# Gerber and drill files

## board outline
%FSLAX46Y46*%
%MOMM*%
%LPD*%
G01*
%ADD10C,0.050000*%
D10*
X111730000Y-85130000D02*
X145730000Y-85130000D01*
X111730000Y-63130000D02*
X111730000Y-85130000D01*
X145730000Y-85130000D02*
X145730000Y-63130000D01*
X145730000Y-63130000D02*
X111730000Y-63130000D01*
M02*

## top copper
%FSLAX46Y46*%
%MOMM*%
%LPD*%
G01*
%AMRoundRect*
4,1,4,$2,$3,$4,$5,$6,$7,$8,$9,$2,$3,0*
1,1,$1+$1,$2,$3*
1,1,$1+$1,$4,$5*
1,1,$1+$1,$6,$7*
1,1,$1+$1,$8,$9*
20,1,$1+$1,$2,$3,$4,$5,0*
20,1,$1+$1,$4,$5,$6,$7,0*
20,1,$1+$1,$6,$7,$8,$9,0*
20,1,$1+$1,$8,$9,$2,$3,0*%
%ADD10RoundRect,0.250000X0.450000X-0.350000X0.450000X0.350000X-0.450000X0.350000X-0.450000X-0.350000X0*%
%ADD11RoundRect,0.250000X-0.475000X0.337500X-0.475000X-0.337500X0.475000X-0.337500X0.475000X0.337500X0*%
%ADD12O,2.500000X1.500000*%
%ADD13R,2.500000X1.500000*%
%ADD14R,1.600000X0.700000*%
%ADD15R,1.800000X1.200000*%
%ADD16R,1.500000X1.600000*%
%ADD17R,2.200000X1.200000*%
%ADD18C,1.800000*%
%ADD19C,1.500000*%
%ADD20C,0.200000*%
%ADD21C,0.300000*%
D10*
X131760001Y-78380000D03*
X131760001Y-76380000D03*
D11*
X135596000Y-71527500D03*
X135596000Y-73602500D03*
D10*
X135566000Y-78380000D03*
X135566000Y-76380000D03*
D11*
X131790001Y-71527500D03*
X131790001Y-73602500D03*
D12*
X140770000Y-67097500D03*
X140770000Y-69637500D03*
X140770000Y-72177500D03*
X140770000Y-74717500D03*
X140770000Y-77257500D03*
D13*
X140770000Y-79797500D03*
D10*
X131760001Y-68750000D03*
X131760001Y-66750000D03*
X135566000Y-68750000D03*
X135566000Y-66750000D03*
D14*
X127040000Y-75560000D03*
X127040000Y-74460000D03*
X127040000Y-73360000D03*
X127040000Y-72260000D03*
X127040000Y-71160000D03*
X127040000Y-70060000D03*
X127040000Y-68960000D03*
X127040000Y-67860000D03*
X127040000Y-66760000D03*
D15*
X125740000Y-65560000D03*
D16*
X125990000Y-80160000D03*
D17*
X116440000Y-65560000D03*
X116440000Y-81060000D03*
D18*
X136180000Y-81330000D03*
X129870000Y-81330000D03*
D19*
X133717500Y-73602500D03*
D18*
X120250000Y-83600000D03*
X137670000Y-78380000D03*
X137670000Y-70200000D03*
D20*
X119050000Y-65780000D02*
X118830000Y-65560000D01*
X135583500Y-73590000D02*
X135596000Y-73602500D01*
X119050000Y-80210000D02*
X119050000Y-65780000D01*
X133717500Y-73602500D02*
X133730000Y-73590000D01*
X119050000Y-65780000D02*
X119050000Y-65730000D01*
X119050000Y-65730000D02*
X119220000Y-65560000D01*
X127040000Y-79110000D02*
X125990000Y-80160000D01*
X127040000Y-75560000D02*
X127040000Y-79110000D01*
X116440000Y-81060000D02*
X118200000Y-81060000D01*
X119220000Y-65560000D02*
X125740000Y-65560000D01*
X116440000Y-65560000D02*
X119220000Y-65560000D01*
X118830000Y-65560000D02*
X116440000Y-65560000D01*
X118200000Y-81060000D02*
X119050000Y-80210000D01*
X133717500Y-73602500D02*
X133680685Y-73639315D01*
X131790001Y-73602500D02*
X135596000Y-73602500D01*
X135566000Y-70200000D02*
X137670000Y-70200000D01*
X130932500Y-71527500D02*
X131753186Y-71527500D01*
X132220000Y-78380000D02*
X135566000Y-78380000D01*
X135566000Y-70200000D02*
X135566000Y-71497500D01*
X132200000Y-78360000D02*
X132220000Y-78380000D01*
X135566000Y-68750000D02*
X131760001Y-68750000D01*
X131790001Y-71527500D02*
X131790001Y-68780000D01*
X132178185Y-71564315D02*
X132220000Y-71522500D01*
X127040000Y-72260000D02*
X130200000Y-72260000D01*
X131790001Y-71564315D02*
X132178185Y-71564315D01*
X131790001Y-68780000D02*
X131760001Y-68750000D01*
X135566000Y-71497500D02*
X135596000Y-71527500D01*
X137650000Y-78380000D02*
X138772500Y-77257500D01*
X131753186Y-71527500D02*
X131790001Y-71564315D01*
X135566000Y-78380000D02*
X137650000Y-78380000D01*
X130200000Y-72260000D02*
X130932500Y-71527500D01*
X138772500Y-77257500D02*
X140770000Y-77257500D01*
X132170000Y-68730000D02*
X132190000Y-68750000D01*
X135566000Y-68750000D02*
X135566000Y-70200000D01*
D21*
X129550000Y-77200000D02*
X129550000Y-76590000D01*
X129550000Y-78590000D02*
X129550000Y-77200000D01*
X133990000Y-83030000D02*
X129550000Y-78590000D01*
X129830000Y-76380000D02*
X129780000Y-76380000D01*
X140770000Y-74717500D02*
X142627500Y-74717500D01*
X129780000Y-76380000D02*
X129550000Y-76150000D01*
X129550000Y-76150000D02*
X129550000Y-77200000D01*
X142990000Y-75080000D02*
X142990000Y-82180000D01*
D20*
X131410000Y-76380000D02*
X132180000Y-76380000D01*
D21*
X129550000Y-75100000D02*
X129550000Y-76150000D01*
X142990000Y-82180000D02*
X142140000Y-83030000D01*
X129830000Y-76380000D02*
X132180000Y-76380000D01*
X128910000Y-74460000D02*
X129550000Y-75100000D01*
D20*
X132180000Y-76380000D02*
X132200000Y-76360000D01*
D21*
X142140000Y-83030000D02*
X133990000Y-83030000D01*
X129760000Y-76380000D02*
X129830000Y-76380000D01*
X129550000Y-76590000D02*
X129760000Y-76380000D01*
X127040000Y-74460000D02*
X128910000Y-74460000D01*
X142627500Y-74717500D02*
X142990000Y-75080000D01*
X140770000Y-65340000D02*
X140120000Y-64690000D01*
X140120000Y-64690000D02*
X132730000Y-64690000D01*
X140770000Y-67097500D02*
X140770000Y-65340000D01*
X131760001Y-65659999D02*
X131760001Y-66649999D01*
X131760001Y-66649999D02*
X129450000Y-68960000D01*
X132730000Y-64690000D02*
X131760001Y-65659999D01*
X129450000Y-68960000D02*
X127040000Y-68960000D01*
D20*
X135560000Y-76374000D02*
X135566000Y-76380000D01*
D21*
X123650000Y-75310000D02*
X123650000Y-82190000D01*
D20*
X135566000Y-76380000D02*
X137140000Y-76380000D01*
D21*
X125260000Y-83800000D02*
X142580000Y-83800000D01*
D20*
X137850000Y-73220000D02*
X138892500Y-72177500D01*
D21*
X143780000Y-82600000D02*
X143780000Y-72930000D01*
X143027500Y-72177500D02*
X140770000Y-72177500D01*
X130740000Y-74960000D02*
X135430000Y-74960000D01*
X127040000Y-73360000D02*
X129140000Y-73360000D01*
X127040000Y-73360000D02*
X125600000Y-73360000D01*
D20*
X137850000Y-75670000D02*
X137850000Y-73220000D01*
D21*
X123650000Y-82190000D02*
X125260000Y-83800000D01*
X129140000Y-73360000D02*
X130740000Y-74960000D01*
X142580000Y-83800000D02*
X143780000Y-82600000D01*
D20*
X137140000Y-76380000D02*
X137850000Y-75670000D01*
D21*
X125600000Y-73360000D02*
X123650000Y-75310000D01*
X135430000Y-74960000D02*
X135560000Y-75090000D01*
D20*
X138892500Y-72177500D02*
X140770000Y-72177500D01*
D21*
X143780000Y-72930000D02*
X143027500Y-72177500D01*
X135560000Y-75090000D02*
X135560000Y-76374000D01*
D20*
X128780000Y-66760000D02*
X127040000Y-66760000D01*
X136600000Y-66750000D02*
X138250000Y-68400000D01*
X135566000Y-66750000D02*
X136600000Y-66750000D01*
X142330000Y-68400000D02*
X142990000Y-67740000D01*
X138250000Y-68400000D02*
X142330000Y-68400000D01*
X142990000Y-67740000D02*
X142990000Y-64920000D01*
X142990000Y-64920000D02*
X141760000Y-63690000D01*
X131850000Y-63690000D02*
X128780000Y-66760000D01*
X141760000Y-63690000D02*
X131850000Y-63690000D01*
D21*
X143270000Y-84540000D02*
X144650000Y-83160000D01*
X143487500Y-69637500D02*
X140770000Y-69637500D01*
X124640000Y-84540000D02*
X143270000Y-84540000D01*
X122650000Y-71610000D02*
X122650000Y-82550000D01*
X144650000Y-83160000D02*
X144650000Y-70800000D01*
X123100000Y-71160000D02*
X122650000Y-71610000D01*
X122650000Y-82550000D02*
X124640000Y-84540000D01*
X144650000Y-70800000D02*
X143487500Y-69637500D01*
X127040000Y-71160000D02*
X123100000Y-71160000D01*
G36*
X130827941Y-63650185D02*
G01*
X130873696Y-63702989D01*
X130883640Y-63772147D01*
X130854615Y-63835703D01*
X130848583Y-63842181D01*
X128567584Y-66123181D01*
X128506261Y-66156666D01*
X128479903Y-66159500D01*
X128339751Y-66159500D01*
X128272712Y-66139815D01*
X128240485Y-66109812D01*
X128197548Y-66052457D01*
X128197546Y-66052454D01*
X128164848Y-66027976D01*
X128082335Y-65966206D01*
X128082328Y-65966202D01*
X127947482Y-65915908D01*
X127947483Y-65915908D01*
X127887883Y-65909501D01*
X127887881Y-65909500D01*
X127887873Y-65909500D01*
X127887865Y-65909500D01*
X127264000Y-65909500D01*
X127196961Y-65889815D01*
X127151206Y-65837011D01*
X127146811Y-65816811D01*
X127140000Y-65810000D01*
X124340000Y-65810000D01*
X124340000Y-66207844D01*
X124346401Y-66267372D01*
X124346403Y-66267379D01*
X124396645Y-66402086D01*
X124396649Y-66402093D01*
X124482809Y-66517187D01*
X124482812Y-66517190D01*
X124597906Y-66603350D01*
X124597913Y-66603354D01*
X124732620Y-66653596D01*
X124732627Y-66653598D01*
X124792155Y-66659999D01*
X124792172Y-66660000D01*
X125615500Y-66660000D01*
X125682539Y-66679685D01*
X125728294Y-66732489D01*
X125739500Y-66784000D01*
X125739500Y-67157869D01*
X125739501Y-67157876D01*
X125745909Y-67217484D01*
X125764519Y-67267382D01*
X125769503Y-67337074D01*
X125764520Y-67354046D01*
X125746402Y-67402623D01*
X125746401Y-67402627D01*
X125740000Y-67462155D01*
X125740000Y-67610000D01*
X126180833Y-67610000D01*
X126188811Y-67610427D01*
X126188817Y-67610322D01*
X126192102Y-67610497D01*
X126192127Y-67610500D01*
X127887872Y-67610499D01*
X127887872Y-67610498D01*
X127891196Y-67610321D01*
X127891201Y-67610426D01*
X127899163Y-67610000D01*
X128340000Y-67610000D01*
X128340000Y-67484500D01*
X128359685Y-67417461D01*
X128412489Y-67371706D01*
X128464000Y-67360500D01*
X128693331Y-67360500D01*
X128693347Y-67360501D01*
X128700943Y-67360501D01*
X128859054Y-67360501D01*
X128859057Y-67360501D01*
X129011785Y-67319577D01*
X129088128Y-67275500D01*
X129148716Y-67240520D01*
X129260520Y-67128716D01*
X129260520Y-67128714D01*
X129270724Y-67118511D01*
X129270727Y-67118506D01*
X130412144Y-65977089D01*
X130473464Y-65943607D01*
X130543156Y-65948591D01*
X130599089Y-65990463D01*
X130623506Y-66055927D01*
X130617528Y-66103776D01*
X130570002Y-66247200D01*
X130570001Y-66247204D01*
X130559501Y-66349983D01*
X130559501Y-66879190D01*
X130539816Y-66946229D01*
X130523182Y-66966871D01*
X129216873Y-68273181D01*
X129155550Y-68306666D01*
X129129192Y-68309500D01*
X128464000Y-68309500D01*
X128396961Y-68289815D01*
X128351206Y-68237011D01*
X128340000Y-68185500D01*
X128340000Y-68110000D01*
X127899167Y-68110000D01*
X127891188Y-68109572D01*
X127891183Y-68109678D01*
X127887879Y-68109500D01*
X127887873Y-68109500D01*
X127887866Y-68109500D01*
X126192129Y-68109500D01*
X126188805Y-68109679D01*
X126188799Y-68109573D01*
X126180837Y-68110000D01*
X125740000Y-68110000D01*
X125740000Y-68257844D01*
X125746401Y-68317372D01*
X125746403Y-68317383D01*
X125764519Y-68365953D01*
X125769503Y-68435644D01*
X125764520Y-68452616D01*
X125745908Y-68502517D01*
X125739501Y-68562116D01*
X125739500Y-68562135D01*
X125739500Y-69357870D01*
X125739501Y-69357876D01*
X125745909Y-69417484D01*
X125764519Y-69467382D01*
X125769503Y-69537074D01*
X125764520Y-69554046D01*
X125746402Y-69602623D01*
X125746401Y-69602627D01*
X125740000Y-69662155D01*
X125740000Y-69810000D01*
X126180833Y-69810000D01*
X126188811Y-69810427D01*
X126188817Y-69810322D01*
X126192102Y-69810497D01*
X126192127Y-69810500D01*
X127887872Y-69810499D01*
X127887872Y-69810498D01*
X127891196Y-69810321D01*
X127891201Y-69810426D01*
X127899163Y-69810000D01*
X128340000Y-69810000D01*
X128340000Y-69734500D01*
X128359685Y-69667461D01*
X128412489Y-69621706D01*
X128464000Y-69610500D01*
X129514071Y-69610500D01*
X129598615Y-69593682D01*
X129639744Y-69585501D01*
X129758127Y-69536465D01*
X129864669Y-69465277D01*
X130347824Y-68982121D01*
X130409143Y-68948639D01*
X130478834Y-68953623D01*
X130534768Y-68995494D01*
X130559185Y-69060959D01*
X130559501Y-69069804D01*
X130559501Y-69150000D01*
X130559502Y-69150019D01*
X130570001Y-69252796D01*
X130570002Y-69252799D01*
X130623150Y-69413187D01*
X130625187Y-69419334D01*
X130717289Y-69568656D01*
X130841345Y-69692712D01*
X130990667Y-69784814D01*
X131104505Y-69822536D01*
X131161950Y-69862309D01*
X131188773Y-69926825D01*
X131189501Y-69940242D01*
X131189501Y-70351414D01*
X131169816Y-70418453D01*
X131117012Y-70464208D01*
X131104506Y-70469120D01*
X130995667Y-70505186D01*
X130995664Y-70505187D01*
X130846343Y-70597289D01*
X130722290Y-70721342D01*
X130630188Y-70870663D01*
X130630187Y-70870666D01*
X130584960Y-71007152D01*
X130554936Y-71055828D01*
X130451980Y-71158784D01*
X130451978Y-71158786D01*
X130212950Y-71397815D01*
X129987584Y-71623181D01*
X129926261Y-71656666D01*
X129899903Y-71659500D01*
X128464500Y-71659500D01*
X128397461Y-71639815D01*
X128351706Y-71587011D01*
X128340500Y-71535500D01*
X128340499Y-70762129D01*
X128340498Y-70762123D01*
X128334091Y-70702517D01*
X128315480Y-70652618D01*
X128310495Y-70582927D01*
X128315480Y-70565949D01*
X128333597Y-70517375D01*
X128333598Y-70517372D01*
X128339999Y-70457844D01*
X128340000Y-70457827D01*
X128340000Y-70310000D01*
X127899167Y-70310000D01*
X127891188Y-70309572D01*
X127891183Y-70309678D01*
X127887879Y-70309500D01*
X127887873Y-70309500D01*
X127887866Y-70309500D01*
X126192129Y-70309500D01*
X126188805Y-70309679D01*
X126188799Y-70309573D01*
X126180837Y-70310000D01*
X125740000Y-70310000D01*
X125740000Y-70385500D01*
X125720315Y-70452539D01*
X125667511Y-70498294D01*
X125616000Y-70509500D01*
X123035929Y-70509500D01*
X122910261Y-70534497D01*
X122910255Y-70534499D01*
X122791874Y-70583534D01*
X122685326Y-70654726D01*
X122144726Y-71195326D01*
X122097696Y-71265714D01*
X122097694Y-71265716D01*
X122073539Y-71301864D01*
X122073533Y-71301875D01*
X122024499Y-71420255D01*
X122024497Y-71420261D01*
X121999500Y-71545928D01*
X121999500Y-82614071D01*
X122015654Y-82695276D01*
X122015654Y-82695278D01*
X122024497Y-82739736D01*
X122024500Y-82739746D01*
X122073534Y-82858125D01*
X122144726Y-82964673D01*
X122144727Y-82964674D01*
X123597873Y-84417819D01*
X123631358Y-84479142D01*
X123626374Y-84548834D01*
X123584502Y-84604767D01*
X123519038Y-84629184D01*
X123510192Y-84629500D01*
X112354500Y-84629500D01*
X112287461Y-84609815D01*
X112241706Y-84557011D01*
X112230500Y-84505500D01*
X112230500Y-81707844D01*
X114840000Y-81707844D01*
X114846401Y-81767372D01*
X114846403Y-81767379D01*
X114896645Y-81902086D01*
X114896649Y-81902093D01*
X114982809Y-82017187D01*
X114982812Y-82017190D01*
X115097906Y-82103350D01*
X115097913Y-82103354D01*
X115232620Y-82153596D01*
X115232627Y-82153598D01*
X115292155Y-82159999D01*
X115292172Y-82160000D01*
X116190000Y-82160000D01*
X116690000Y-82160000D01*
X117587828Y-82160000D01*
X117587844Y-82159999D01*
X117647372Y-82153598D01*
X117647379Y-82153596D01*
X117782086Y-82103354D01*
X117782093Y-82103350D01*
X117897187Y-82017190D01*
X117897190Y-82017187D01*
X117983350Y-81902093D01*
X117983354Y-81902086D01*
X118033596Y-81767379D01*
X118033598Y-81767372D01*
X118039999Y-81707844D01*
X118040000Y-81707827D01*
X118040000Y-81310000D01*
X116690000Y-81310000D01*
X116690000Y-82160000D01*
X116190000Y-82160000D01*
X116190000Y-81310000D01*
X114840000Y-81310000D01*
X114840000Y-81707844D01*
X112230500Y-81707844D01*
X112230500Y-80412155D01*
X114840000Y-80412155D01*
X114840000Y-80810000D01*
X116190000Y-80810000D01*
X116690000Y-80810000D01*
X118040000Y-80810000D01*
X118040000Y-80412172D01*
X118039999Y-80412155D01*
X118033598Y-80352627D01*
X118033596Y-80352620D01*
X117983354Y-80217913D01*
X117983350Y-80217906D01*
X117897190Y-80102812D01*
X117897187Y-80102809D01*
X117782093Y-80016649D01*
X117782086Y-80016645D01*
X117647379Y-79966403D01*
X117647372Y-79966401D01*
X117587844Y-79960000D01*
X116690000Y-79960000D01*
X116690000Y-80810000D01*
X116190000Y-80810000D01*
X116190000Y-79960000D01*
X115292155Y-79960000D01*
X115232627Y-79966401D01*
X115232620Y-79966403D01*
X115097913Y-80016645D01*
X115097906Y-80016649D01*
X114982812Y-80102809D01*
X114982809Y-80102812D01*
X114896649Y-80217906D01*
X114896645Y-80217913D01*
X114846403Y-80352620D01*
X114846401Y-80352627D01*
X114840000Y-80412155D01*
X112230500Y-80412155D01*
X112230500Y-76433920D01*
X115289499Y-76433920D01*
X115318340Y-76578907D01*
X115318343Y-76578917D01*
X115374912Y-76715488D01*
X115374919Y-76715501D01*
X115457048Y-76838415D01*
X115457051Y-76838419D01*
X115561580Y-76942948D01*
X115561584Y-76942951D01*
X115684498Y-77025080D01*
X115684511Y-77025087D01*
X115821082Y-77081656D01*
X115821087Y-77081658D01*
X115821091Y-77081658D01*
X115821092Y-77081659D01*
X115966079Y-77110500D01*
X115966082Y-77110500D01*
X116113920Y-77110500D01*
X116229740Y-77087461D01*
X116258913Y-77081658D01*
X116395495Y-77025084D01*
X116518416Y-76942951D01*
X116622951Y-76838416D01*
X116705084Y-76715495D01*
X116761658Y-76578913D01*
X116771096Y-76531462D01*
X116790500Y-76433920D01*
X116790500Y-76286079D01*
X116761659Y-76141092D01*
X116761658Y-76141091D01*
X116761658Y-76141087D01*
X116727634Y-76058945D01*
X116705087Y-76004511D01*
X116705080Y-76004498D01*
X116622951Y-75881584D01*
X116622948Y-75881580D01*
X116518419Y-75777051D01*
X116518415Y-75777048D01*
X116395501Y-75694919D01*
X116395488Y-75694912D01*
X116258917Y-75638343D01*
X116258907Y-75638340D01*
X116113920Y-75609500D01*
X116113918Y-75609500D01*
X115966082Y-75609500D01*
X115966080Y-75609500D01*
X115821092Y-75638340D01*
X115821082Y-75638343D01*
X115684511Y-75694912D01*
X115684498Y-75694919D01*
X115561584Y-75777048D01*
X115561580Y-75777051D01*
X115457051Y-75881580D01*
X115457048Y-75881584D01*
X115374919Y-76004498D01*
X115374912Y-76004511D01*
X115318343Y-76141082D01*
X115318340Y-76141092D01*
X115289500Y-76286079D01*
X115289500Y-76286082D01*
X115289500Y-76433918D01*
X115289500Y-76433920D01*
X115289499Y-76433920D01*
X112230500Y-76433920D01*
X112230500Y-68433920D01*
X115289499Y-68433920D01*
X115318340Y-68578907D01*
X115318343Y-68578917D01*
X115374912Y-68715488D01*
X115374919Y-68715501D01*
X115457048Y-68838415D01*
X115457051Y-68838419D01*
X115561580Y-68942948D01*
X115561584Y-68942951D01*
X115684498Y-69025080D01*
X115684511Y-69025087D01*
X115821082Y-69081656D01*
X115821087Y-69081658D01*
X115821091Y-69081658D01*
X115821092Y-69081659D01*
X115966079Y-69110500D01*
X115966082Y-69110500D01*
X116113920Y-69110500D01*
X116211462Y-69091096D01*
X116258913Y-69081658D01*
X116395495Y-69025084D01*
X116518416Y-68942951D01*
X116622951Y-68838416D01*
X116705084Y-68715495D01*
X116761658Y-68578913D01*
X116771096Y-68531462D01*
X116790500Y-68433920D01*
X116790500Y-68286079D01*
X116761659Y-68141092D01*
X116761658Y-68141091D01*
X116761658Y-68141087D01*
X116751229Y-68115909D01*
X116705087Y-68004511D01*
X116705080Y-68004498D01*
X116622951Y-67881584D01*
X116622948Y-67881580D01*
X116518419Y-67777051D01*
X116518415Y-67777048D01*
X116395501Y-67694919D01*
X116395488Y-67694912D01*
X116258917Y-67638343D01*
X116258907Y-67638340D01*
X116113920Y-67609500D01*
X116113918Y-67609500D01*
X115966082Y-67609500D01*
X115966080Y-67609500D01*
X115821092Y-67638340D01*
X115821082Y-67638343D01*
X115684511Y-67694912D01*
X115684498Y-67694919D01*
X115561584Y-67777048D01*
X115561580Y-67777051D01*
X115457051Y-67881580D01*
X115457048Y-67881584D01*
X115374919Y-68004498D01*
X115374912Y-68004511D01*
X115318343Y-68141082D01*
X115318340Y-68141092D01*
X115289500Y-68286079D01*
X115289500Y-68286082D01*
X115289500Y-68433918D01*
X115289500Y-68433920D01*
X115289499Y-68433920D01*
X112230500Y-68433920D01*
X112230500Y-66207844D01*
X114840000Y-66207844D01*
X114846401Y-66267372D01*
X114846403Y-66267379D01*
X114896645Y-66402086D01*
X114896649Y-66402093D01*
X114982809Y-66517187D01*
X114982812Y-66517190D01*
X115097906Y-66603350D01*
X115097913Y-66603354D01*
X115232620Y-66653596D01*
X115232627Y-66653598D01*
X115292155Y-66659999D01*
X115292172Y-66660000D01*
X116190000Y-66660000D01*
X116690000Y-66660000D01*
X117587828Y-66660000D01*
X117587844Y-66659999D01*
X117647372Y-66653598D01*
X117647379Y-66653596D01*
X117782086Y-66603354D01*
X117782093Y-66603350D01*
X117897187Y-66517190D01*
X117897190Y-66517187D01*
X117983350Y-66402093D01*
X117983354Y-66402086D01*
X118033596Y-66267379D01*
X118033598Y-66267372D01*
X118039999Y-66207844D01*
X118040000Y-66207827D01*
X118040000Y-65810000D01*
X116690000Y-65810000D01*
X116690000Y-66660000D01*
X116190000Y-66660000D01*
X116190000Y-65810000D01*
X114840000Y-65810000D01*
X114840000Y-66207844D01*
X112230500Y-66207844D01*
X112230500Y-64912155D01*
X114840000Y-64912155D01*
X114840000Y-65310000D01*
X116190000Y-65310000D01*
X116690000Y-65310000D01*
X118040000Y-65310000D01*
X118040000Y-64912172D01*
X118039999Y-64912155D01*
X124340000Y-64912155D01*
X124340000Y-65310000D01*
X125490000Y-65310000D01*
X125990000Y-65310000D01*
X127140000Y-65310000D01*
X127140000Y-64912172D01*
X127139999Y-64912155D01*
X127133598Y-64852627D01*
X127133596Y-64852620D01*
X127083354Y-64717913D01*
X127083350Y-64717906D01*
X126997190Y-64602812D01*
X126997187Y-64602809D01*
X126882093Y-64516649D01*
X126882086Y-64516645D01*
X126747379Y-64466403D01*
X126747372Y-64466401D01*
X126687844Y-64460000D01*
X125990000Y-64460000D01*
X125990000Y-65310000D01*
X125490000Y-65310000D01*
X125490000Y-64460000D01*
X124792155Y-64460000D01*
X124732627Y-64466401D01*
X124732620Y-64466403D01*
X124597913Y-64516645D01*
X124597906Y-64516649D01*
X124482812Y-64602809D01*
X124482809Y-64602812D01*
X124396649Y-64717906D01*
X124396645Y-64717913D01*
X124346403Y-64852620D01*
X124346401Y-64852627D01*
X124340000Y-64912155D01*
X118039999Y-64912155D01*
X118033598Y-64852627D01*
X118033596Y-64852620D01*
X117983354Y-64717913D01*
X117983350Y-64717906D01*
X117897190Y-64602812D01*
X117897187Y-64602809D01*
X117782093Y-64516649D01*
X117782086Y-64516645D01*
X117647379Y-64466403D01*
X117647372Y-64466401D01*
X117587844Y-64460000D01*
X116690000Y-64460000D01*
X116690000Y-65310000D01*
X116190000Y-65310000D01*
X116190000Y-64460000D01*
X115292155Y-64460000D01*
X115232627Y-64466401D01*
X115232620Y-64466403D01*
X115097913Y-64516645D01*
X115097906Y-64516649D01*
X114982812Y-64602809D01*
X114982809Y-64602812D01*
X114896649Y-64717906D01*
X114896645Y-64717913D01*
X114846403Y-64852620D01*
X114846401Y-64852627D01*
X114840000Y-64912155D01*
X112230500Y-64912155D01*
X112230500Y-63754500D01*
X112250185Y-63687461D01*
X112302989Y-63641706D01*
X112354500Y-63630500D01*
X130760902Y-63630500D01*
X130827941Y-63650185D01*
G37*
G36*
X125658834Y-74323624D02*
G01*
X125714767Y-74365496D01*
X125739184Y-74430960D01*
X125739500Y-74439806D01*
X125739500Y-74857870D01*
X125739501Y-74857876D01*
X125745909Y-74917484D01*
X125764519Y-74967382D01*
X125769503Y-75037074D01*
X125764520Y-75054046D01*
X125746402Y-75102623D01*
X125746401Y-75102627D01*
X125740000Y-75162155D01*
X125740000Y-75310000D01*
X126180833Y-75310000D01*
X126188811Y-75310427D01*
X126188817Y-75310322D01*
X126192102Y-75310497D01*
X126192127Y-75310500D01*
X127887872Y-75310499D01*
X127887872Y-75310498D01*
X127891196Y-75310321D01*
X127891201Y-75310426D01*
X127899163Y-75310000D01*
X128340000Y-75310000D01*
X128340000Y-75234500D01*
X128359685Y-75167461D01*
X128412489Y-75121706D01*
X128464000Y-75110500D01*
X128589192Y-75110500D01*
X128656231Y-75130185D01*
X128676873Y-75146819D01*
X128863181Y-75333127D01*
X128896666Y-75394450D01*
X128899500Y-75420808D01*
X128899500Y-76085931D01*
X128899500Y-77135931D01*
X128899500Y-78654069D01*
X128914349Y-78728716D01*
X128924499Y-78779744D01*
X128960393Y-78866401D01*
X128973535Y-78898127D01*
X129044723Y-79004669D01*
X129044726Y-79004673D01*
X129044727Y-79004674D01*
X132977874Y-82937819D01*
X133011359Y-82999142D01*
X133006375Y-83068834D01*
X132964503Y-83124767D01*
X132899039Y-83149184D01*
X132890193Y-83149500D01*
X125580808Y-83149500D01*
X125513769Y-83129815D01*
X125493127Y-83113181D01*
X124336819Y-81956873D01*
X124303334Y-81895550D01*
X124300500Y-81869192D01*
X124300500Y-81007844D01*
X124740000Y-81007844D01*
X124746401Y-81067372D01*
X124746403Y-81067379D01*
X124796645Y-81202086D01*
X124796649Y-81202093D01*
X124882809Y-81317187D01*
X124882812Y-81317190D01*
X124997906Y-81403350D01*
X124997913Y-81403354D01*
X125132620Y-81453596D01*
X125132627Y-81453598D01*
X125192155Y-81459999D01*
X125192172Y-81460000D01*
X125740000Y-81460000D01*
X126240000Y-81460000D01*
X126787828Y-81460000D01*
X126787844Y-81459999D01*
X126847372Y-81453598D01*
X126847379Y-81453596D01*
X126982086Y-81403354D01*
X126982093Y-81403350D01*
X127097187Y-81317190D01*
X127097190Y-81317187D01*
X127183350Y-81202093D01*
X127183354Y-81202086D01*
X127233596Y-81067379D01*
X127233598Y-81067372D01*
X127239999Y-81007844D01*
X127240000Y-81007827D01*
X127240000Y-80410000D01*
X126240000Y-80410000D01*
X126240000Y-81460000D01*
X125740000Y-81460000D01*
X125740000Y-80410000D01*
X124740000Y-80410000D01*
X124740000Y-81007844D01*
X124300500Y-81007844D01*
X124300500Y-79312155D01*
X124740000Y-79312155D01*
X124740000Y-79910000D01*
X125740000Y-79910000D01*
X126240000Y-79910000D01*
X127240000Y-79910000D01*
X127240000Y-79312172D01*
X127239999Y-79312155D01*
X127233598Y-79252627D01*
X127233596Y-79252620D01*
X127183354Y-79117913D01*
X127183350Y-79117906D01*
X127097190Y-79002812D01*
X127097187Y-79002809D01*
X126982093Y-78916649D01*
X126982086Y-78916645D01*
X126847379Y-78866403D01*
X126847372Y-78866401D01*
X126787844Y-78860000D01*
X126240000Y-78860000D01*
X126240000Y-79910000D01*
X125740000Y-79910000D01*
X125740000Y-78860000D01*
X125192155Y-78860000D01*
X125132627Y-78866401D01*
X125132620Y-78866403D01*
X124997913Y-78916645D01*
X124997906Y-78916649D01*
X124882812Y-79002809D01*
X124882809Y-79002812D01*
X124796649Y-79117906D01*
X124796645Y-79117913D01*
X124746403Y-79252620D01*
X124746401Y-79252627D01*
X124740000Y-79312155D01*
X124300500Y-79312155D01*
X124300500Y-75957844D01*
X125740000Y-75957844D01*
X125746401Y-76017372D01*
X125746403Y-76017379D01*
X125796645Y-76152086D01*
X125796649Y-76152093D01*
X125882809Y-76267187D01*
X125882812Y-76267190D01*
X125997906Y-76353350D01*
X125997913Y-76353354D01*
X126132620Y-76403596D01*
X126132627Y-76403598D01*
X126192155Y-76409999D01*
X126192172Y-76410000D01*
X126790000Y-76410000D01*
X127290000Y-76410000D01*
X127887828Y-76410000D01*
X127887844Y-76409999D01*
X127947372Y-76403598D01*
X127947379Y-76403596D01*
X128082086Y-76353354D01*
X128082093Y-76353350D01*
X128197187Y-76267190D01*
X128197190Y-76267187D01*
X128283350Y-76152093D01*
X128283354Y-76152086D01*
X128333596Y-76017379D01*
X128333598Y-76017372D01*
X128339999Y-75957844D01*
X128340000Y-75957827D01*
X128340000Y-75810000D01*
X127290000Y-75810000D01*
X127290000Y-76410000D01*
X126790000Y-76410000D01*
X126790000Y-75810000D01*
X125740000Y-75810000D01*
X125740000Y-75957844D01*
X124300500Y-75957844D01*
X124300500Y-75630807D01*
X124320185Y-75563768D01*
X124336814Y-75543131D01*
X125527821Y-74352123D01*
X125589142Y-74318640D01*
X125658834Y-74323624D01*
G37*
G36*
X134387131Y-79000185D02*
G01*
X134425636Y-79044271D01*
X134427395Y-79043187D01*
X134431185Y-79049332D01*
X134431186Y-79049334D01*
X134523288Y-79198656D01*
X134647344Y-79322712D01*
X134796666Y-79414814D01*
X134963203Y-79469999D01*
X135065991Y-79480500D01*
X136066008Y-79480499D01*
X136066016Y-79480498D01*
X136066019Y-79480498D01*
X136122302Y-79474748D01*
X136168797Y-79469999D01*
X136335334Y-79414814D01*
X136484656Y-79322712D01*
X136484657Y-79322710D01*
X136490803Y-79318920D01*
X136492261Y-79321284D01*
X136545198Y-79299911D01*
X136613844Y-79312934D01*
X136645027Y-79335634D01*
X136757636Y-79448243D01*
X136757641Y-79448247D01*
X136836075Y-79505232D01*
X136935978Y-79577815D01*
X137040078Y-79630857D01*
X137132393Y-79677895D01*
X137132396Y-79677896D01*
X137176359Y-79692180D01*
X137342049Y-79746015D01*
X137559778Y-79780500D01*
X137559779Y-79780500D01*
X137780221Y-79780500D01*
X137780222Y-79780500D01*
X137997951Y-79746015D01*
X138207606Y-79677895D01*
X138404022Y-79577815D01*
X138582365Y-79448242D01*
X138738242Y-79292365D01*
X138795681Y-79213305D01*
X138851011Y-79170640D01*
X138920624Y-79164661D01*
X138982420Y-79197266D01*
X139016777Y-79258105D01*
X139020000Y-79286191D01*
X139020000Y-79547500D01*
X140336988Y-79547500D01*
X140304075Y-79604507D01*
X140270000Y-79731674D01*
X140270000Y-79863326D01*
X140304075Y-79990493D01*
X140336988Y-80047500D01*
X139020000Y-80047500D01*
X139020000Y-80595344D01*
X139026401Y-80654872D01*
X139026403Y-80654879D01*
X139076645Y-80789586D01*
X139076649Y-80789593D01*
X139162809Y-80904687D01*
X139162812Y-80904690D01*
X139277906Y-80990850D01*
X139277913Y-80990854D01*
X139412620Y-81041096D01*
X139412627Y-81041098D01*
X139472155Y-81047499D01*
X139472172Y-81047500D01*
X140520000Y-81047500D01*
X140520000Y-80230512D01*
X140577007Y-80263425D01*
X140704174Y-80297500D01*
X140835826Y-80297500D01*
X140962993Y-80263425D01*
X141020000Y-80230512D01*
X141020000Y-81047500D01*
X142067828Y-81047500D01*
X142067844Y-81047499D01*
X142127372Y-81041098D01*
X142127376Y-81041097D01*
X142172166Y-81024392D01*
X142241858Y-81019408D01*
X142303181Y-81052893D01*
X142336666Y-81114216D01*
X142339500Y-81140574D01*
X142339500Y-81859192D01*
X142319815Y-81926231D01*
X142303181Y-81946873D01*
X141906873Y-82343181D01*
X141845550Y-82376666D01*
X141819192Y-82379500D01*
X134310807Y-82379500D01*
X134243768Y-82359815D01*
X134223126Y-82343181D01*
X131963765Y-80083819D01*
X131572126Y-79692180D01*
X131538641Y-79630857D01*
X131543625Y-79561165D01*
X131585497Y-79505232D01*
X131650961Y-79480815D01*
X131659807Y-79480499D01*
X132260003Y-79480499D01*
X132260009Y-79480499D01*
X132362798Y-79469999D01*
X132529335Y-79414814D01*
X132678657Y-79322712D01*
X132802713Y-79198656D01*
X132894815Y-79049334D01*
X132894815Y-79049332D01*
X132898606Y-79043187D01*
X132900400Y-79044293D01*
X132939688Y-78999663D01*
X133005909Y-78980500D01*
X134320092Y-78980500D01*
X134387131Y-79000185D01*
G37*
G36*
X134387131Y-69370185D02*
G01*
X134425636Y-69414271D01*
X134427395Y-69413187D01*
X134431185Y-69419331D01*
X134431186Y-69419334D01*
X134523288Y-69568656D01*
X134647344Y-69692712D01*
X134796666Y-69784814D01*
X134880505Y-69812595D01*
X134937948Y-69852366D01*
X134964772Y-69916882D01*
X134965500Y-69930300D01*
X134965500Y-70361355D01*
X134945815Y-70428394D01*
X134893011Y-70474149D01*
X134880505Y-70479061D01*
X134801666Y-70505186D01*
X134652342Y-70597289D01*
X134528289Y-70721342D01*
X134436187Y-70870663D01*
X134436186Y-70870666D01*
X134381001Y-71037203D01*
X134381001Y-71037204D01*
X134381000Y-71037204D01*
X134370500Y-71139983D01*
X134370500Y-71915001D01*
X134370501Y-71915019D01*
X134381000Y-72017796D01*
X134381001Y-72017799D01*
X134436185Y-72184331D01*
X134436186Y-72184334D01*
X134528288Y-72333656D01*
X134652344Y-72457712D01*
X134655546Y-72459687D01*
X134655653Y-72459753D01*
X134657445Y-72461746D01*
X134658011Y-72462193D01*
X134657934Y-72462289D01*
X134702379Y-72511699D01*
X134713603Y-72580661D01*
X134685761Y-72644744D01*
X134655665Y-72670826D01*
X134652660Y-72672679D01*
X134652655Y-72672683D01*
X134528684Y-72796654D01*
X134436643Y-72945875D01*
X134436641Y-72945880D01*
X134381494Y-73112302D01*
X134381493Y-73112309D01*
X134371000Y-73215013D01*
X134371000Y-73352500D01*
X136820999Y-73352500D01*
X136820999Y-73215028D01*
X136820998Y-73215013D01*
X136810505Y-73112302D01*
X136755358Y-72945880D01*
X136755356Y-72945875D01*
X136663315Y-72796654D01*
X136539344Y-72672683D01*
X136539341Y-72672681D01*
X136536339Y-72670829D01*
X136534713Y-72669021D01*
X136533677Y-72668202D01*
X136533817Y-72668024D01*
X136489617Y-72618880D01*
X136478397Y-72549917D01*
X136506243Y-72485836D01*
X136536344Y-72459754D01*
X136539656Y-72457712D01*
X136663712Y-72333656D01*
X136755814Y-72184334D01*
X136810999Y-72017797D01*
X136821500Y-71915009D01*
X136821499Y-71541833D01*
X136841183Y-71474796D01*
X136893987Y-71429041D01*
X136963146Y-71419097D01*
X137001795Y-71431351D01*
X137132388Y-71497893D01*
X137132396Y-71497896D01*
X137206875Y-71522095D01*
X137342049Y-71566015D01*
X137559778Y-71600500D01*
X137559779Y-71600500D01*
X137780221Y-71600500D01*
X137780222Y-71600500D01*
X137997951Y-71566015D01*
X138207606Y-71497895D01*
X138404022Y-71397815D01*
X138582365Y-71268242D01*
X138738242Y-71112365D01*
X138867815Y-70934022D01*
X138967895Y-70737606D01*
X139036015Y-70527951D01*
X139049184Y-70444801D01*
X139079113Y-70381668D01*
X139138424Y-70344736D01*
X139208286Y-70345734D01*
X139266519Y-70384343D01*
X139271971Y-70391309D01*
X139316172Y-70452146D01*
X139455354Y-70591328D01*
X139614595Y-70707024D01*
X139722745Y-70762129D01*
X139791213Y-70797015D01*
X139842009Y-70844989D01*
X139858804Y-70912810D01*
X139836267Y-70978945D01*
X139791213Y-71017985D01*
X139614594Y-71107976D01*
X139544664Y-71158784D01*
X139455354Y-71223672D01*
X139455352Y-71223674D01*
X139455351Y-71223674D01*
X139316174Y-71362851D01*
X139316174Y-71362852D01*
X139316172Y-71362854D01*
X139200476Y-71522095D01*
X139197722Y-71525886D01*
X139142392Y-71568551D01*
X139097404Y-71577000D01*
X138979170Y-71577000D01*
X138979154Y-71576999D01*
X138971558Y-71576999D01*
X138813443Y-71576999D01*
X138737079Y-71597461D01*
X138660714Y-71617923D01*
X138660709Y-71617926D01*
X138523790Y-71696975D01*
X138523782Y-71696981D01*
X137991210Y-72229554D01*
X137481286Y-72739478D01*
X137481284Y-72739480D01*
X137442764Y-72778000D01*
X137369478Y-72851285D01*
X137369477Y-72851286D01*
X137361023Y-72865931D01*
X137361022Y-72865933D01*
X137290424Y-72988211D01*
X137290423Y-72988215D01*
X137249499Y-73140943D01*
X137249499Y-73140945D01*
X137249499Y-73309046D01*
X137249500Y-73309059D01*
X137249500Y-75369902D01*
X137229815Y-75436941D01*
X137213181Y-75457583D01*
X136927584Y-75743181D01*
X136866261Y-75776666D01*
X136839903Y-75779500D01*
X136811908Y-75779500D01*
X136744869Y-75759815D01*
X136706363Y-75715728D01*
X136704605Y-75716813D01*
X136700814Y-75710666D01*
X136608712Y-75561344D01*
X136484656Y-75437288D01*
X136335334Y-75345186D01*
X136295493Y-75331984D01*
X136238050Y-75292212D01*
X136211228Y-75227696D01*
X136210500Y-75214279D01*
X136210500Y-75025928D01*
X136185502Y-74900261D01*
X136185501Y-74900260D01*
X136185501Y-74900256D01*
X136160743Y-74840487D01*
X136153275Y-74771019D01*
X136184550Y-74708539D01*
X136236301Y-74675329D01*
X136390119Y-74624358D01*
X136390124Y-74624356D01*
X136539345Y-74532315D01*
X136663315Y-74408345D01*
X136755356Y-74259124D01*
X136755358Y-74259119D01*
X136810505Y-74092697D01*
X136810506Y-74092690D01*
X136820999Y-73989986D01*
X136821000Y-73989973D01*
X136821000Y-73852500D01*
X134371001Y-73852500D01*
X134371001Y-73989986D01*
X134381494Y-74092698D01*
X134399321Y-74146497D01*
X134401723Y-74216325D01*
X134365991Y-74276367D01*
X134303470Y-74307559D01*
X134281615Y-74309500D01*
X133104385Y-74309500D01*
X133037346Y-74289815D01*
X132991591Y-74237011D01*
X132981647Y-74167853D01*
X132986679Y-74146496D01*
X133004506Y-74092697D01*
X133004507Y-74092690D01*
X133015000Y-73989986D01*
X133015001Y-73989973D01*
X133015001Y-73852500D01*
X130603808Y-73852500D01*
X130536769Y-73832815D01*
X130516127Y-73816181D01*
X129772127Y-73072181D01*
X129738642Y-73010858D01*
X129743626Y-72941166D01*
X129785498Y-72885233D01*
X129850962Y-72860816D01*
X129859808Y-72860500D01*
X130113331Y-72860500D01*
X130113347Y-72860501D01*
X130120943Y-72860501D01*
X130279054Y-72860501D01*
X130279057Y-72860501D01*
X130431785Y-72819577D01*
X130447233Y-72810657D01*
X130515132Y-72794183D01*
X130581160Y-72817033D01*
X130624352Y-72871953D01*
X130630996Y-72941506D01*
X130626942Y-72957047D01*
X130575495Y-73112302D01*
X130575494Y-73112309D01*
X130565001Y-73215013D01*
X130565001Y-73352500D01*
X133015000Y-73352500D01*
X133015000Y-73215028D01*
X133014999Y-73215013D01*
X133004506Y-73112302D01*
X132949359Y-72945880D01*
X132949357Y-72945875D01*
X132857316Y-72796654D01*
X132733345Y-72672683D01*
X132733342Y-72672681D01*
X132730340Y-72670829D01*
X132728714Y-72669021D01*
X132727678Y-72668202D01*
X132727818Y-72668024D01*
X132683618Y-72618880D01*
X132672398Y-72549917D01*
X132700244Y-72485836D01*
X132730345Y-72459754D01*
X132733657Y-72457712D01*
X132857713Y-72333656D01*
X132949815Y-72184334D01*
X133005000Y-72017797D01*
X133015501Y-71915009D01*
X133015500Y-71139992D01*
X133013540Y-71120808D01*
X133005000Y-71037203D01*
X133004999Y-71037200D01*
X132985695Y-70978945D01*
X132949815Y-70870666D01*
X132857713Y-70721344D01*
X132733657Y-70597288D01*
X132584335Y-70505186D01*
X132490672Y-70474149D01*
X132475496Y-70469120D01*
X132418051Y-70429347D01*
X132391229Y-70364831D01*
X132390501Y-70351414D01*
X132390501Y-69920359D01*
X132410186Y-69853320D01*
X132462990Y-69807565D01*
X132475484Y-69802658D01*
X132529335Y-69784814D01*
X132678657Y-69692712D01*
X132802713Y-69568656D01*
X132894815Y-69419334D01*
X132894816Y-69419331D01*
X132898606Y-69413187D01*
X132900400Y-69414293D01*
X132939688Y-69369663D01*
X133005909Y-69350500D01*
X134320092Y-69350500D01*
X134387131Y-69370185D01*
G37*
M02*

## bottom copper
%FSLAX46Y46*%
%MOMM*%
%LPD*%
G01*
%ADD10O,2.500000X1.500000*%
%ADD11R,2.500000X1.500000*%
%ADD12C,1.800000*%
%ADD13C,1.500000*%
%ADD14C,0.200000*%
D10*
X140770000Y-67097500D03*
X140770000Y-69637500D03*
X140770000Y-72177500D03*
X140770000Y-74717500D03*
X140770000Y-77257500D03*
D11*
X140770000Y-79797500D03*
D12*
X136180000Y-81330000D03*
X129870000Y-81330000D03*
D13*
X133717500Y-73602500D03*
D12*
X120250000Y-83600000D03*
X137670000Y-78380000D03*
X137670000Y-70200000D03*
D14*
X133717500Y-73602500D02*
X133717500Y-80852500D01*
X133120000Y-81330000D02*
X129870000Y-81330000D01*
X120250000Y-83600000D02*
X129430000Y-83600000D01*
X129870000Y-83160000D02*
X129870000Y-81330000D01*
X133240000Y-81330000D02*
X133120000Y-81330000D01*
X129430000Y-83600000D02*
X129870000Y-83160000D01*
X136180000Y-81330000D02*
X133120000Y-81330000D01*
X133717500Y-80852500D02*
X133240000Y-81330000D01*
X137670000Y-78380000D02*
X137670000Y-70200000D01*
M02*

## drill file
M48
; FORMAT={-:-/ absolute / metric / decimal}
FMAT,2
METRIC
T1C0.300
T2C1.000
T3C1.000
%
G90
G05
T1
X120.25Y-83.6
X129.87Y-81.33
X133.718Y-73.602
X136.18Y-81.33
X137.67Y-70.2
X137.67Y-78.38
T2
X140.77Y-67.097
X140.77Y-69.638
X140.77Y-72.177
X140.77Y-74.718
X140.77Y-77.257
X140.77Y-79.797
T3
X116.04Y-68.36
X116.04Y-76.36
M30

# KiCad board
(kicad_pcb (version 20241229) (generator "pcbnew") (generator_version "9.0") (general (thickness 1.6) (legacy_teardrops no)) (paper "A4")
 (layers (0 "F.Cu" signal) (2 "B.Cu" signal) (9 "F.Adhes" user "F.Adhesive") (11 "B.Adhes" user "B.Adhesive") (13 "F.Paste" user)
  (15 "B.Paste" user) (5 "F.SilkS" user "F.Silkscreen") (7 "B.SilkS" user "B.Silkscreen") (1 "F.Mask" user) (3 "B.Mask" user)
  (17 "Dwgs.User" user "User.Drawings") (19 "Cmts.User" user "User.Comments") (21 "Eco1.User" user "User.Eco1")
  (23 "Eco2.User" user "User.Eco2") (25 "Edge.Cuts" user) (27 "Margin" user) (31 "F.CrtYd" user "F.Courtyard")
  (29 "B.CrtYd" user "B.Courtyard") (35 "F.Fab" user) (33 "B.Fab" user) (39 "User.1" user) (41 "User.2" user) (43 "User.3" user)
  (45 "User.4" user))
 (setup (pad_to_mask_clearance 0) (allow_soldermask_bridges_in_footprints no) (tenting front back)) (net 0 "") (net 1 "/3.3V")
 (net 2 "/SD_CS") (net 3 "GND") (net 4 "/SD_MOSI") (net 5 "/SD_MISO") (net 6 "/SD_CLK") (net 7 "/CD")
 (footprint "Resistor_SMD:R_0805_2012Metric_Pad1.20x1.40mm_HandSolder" (layer "F.Cu") (at 131.760001 77.38 90)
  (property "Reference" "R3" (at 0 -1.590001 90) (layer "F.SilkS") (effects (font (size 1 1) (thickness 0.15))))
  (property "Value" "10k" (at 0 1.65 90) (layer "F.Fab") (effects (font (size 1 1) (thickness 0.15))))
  (pad "1" smd roundrect (at -1 0 90) (size 1.2 1.4) (layers "F.Cu" "F.Mask" "F.Paste") (roundrect_rratio 0.208333) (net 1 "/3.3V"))
  (pad "2" smd roundrect (at 1 0 90) (size 1.2 1.4) (layers "F.Cu" "F.Mask" "F.Paste") (roundrect_rratio 0.208333) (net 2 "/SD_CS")))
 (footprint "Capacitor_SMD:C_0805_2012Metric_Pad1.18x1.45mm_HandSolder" (layer "F.Cu") (at 135.596 72.565 -90)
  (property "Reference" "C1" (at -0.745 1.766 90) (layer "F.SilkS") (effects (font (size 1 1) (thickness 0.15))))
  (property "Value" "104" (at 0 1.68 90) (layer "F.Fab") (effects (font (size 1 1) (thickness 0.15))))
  (pad "1" smd roundrect (at -1.0375 0 270) (size 1.175 1.45) (layers "F.Cu" "F.Mask" "F.Paste") (roundrect_rratio 0.212766) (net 1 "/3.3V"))
  (pad "2" smd roundrect (at 1.0375 0 270) (size 1.175 1.45) (layers "F.Cu" "F.Mask" "F.Paste") (roundrect_rratio 0.212766) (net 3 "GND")))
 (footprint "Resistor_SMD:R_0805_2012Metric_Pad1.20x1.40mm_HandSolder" (layer "F.Cu") (at 135.566 77.38 90)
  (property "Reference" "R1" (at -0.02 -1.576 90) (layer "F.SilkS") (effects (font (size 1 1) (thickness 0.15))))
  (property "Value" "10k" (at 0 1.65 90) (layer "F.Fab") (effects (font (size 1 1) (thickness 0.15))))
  (pad "1" smd roundrect (at -1 0 90) (size 1.2 1.4) (layers "F.Cu" "F.Mask" "F.Paste") (roundrect_rratio 0.208333) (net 1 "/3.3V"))
  (pad "2" smd roundrect (at 1 0 90) (size 1.2 1.4) (layers "F.Cu" "F.Mask" "F.Paste") (roundrect_rratio 0.208333) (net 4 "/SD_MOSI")))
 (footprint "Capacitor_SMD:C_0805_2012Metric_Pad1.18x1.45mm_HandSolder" (layer "F.Cu") (at 131.790001 72.565 -90)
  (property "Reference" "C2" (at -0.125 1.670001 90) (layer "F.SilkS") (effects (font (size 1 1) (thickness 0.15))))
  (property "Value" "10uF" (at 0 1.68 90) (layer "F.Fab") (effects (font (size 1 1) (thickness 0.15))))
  (pad "1" smd roundrect (at -1.0375 0 270) (size 1.175 1.45) (layers "F.Cu" "F.Mask" "F.Paste") (roundrect_rratio 0.212766) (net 1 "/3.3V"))
  (pad "2" smd roundrect (at 1.0375 0 270) (size 1.175 1.45) (layers "F.Cu" "F.Mask" "F.Paste") (roundrect_rratio 0.212766) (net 3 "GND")))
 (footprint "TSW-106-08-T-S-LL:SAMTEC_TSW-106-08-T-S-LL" (layer "F.Cu") (at 140.77 67.0975 -90)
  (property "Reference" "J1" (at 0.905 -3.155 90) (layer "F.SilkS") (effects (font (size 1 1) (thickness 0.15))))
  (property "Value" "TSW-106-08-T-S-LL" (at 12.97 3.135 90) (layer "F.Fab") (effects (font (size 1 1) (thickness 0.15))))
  (pad "01" thru_hole oval (at 0 0 270) (size 1.5 2.5) (drill 1) (layers "*.Cu" "*.Mask") (remove_unused_layers no) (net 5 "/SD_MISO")
   (solder_mask_margin 0.102))
  (pad "02" thru_hole oval (at 2.54 0 270) (size 1.5 2.5) (drill 1) (layers "*.Cu" "*.Mask") (remove_unused_layers no) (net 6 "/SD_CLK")
   (solder_mask_margin 0.102))
  (pad "03" thru_hole oval (at 5.08 0 270) (size 1.5 2.5) (drill 1) (layers "*.Cu" "*.Mask") (remove_unused_layers no) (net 4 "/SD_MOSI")
   (solder_mask_margin 0.102))
  (pad "04" thru_hole oval (at 7.62 0 270) (size 1.5 2.5) (drill 1) (layers "*.Cu" "*.Mask") (remove_unused_layers no) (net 2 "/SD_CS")
   (solder_mask_margin 0.102))
  (pad "05" thru_hole oval (at 10.16 0 270) (size 1.5 2.5) (drill 1) (layers "*.Cu" "*.Mask") (remove_unused_layers no) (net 1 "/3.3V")
   (solder_mask_margin 0.102))
  (pad "06" thru_hole rect (at 12.7 0 270) (size 1.5 2.5) (drill 1) (layers "*.Cu" "*.Mask") (remove_unused_layers no) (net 3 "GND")
   (solder_mask_margin 0.102)))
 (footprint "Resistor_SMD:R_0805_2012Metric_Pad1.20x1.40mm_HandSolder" (layer "F.Cu") (at 131.760001 67.75 90)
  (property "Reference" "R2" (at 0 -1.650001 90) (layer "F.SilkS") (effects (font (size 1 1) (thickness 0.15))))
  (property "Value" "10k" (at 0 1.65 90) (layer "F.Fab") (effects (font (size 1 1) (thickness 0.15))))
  (pad "1" smd roundrect (at -1 0 90) (size 1.2 1.4) (layers "F.Cu" "F.Mask" "F.Paste") (roundrect_rratio 0.208333) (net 1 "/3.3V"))
  (pad "2" smd roundrect (at 1 0 90) (size 1.2 1.4) (layers "F.Cu" "F.Mask" "F.Paste") (roundrect_rratio 0.208333) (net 5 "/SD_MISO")))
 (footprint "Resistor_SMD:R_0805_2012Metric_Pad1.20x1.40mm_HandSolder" (layer "F.Cu") (at 135.566 67.75 90)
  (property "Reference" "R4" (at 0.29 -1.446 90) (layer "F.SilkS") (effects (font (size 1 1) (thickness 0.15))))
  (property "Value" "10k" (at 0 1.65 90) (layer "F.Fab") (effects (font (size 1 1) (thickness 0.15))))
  (pad "1" smd roundrect (at -1 0 90) (size 1.2 1.4) (layers "F.Cu" "F.Mask" "F.Paste") (roundrect_rratio 0.208333) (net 1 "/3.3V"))
  (pad "2" smd roundrect (at 1 0 90) (size 1.2 1.4) (layers "F.Cu" "F.Mask" "F.Paste") (roundrect_rratio 0.208333) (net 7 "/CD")))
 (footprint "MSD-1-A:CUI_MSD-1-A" (layer "F.Cu") (at 119.29 73.31 -90)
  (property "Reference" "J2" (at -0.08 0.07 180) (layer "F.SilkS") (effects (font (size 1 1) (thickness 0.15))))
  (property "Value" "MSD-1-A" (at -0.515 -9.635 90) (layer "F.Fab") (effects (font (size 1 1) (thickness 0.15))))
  (pad "" np_thru_hole circle (at -4.95 3.25 270) (size 1 1) (drill 1) (layers "*.Cu" "*.Mask"))
  (pad "" np_thru_hole circle (at 3.05 3.25 270) (size 1 1) (drill 1) (layers "*.Cu" "*.Mask"))
  (pad "1" smd rect (at 2.25 -7.75 270) (size 0.7 1.6) (layers "F.Cu" "F.Mask" "F.Paste") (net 3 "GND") (solder_mask_margin 0.102))
  (pad "2" smd rect (at 1.15 -7.75 270) (size 0.7 1.6) (layers "F.Cu" "F.Mask" "F.Paste") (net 2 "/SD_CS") (solder_mask_margin 0.102))
  (pad "3" smd rect (at 0.05 -7.75 270) (size 0.7 1.6) (layers "F.Cu" "F.Mask" "F.Paste") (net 4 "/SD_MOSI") (solder_mask_margin 0.102))
  (pad "4" smd rect (at -1.05 -7.75 270) (size 0.7 1.6) (layers "F.Cu" "F.Mask" "F.Paste") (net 1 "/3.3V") (solder_mask_margin 0.102))
  (pad "5" smd rect (at -2.15 -7.75 270) (size 0.7 1.6) (layers "F.Cu" "F.Mask" "F.Paste") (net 6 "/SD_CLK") (solder_mask_margin 0.102))
  (pad "6" smd rect (at -3.25 -7.75 270) (size 0.7 1.6) (layers "F.Cu" "F.Mask" "F.Paste") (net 3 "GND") (solder_mask_margin 0.102))
  (pad "7" smd rect (at -4.35 -7.75 270) (size 0.7 1.6) (layers "F.Cu" "F.Mask" "F.Paste") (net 5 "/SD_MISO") (solder_mask_margin 0.102))
  (pad "8" smd rect (at -5.45 -7.75 270) (size 0.7 1.6) (layers "F.Cu" "F.Mask" "F.Paste") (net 3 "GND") (solder_mask_margin 0.102))
  (pad "CD" smd rect (at -6.55 -7.75 270) (size 0.7 1.6) (layers "F.Cu" "F.Mask" "F.Paste") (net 7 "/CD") (solder_mask_margin 0.102))
  (pad "G1" smd rect (at -7.75 -6.45 270) (size 1.2 1.8) (layers "F.Cu" "F.Mask" "F.Paste") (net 3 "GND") (solder_mask_margin 0.102))
  (pad "G2" smd rect (at 6.85 -6.7 270) (size 1.6 1.5) (layers "F.Cu" "F.Mask" "F.Paste") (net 3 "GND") (solder_mask_margin 0.102))
  (pad "G3" smd rect (at -7.75 2.85 270) (size 1.2 2.2) (layers "F.Cu" "F.Mask" "F.Paste") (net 3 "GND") (solder_mask_margin 0.102))
  (pad "G4" smd rect (at 7.75 2.85 270) (size 1.2 2.2) (layers "F.Cu" "F.Mask" "F.Paste") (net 3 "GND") (solder_mask_margin 0.102)))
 (gr_line (start 111.73 85.13) (end 145.73 85.13) (stroke (width 0.05) (type default)) (layer "Edge.Cuts"))
 (gr_line (start 111.73 63.13) (end 111.73 85.13) (stroke (width 0.05) (type default)) (layer "Edge.Cuts"))
 (gr_line (start 145.73 85.13) (end 145.73 63.13) (stroke (width 0.05) (type default)) (layer "Edge.Cuts"))
 (gr_line (start 145.73 63.13) (end 111.73 63.13) (stroke (width 0.05) (type default)) (layer "Edge.Cuts"))
 (segment (start 119.05 65.78) (end 118.83 65.56) (width 0.2) (layer "F.Cu") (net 3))
 (segment (start 135.5835 73.59) (end 135.596 73.6025) (width 0.2) (layer "F.Cu") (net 3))
 (segment (start 119.05 80.21) (end 119.05 65.78) (width 0.2) (layer "F.Cu") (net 3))
 (segment (start 133.7175 73.6025) (end 133.73 73.59) (width 0.2) (layer "F.Cu") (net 3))
 (segment (start 119.05 65.78) (end 119.05 65.73) (width 0.2) (layer "F.Cu") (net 3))
 (segment (start 119.05 65.73) (end 119.22 65.56) (width 0.2) (layer "F.Cu") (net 3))
 (segment (start 127.04 79.11) (end 125.99 80.16) (width 0.2) (layer "F.Cu") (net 3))
 (segment (start 127.04 75.56) (end 127.04 79.11) (width 0.2) (layer "F.Cu") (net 3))
 (segment (start 116.44 81.06) (end 118.2 81.06) (width 0.2) (layer "F.Cu") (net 3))
 (segment (start 119.22 65.56) (end 125.74 65.56) (width 0.2) (layer "F.Cu") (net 3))
 (segment (start 116.44 65.56) (end 119.22 65.56) (width 0.2) (layer "F.Cu") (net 3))
 (segment (start 118.83 65.56) (end 116.44 65.56) (width 0.2) (layer "F.Cu") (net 3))
 (segment (start 118.2 81.06) (end 119.05 80.21) (width 0.2) (layer "F.Cu") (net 3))
 (segment (start 133.7175 73.6025) (end 133.680685 73.639315) (width 0.2) (layer "F.Cu") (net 3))
 (segment (start 131.790001 73.6025) (end 135.596 73.6025) (width 0.2) (layer "F.Cu") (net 3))
 (via (at 136.18 81.33) (size 1.8) (drill 0.3) (layers "F.Cu" "B.Cu") (free yes) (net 3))
 (via (at 129.87 81.33) (size 1.8) (drill 0.3) (layers "F.Cu" "B.Cu") (free yes) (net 3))
 (via (at 133.7175 73.6025) (size 1.5) (drill 0.3) (layers "F.Cu" "B.Cu") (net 3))
 (via (at 120.25 83.6) (size 1.8) (drill 0.3) (layers "F.Cu" "B.Cu") (free yes) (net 3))
 (segment (start 133.7175 73.6025) (end 133.7175 80.8525) (width 0.2) (layer "B.Cu") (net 3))
 (segment (start 133.12 81.33) (end 129.87 81.33) (width 0.2) (layer "B.Cu") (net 3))
 (segment (start 120.25 83.6) (end 129.43 83.6) (width 0.2) (layer "B.Cu") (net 3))
 (segment (start 129.87 83.16) (end 129.87 81.33) (width 0.2) (layer "B.Cu") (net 3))
 (segment (start 133.24 81.33) (end 133.12 81.33) (width 0.2) (layer "B.Cu") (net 3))
 (segment (start 129.43 83.6) (end 129.87 83.16) (width 0.2) (layer "B.Cu") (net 3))
 (segment (start 136.18 81.33) (end 133.12 81.33) (width 0.2) (layer "B.Cu") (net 3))
 (segment (start 133.7175 80.8525) (end 133.24 81.33) (width 0.2) (layer "B.Cu") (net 3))
 (segment (start 135.566 70.2) (end 137.67 70.2) (width 0.2) (layer "F.Cu") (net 1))
 (segment (start 130.9325 71.5275) (end 131.753186 71.5275) (width 0.2) (layer "F.Cu") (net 1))
 (segment (start 132.22 78.38) (end 135.566 78.38) (width 0.2) (layer "F.Cu") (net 1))
 (segment (start 135.566 70.2) (end 135.566 71.4975) (width 0.2) (layer "F.Cu") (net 1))
 (segment (start 132.2 78.36) (end 132.22 78.38) (width 0.2) (layer "F.Cu") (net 1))
 (segment (start 135.566 68.75) (end 131.760001 68.75) (width 0.2) (layer "F.Cu") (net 1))
 (segment (start 131.790001 71.5275) (end 131.790001 68.78) (width 0.2) (layer "F.Cu") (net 1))
 (segment (start 132.178185 71.564315) (end 132.22 71.5225) (width 0.2) (layer "F.Cu") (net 1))
 (segment (start 127.04 72.26) (end 130.2 72.26) (width 0.2) (layer "F.Cu") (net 1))
 (segment (start 131.790001 71.564315) (end 132.178185 71.564315) (width 0.2) (layer "F.Cu") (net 1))
 (segment (start 131.790001 68.78) (end 131.760001 68.75) (width 0.2) (layer "F.Cu") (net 1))
 (segment (start 135.566 71.4975) (end 135.596 71.5275) (width 0.2) (layer "F.Cu") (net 1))
 (segment (start 137.65 78.38) (end 138.7725 77.2575) (width 0.2) (layer "F.Cu") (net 1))
 (segment (start 131.753186 71.5275) (end 131.790001 71.564315) (width 0.2) (layer "F.Cu") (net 1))
 (segment (start 135.566 78.38) (end 137.65 78.38) (width 0.2) (layer "F.Cu") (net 1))
 (segment (start 130.2 72.26) (end 130.9325 71.5275) (width 0.2) (layer "F.Cu") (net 1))
 (segment (start 138.7725 77.2575) (end 140.77 77.2575) (width 0.2) (layer "F.Cu") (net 1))
 (segment (start 132.17 68.73) (end 132.19 68.75) (width 0.2) (layer "F.Cu") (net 1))
 (segment (start 135.566 68.75) (end 135.566 70.2) (width 0.2) (layer "F.Cu") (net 1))
 (via (at 137.67 78.38) (size 1.8) (drill 0.3) (layers "F.Cu" "B.Cu") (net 1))
 (via (at 137.67 70.2) (size 1.8) (drill 0.3) (layers "F.Cu" "B.Cu") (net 1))
 (segment (start 137.67 78.38) (end 137.67 70.2) (width 0.2) (layer "B.Cu") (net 1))
 (segment (start 129.55 77.2) (end 129.55 76.59) (width 0.3) (layer "F.Cu") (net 2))
 (segment (start 129.55 78.59) (end 129.55 77.2) (width 0.3) (layer "F.Cu") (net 2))
 (segment (start 133.99 83.03) (end 129.55 78.59) (width 0.3) (layer "F.Cu") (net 2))
 (segment (start 129.83 76.38) (end 129.78 76.38) (width 0.3) (layer "F.Cu") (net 2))
 (segment (start 140.77 74.7175) (end 142.6275 74.7175) (width 0.3) (layer "F.Cu") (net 2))
 (segment (start 129.78 76.38) (end 129.55 76.15) (width 0.3) (layer "F.Cu") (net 2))
 (segment (start 129.55 76.15) (end 129.55 77.2) (width 0.3) (layer "F.Cu") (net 2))
 (segment (start 142.99 75.08) (end 142.99 82.18) (width 0.3) (layer "F.Cu") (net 2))
 (segment (start 131.41 76.38) (end 132.18 76.38) (width 0.2) (layer "F.Cu") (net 2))
 (segment (start 129.55 75.1) (end 129.55 76.15) (width 0.3) (layer "F.Cu") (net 2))
 (segment (start 142.99 82.18) (end 142.14 83.03) (width 0.3) (layer "F.Cu") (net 2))
 (segment (start 129.83 76.38) (end 132.18 76.38) (width 0.3) (layer "F.Cu") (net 2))
 (segment (start 128.91 74.46) (end 129.55 75.1) (width 0.3) (layer "F.Cu") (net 2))
 (segment (start 132.18 76.38) (end 132.2 76.36) (width 0.2) (layer "F.Cu") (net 2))
 (segment (start 142.14 83.03) (end 133.99 83.03) (width 0.3) (layer "F.Cu") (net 2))
 (segment (start 129.76 76.38) (end 129.83 76.38) (width 0.3) (layer "F.Cu") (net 2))
 (segment (start 129.55 76.59) (end 129.76 76.38) (width 0.3) (layer "F.Cu") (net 2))
 (segment (start 127.04 74.46) (end 128.91 74.46) (width 0.3) (layer "F.Cu") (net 2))
 (segment (start 142.6275 74.7175) (end 142.99 75.08) (width 0.3) (layer "F.Cu") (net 2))
 (segment (start 140.77 65.34) (end 140.12 64.69) (width 0.3) (layer "F.Cu") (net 5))
 (segment (start 140.12 64.69) (end 132.73 64.69) (width 0.3) (layer "F.Cu") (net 5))
 (segment (start 140.77 67.0975) (end 140.77 65.34) (width 0.3) (layer "F.Cu") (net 5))
 (segment (start 131.760001 65.659999) (end 131.760001 66.649999) (width 0.3) (layer "F.Cu") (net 5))
 (segment (start 131.760001 66.649999) (end 129.45 68.96) (width 0.3) (layer "F.Cu") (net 5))
 (segment (start 132.73 64.69) (end 131.760001 65.659999) (width 0.3) (layer "F.Cu") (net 5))
 (segment (start 129.45 68.96) (end 127.04 68.96) (width 0.3) (layer "F.Cu") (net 5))
 (segment (start 135.56 76.374) (end 135.566 76.38) (width 0.2) (layer "F.Cu") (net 4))
 (segment (start 123.65 75.31) (end 123.65 82.19) (width 0.3) (layer "F.Cu") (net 4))
 (segment (start 135.566 76.38) (end 137.14 76.38) (width 0.2) (layer "F.Cu") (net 4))
 (segment (start 125.26 83.8) (end 142.58 83.8) (width 0.3) (layer "F.Cu") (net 4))
 (segment (start 137.85 73.22) (end 138.8925 72.1775) (width 0.2) (layer "F.Cu") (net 4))
 (segment (start 143.78 82.6) (end 143.78 72.93) (width 0.3) (layer "F.Cu") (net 4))
 (segment (start 143.0275 72.1775) (end 140.77 72.1775) (width 0.3) (layer "F.Cu") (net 4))
 (segment (start 130.74 74.96) (end 135.43 74.96) (width 0.3) (layer "F.Cu") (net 4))
 (segment (start 127.04 73.36) (end 129.14 73.36) (width 0.3) (layer "F.Cu") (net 4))
 (segment (start 127.04 73.36) (end 125.6 73.36) (width 0.3) (layer "F.Cu") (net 4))
 (segment (start 137.85 75.67) (end 137.85 73.22) (width 0.2) (layer "F.Cu") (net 4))
 (segment (start 123.65 82.19) (end 125.26 83.8) (width 0.3) (layer "F.Cu") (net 4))
 (segment (start 129.14 73.36) (end 130.74 74.96) (width 0.3) (layer "F.Cu") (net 4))
 (segment (start 142.58 83.8) (end 143.78 82.6) (width 0.3) (layer "F.Cu") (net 4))
 (segment (start 137.14 76.38) (end 137.85 75.67) (width 0.2) (layer "F.Cu") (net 4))
 (segment (start 125.6 73.36) (end 123.65 75.31) (width 0.3) (layer "F.Cu") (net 4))
 (segment (start 135.43 74.96) (end 135.56 75.09) (width 0.3) (layer "F.Cu") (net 4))
 (segment (start 138.8925 72.1775) (end 140.77 72.1775) (width 0.2) (layer "F.Cu") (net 4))
 (segment (start 143.78 72.93) (end 143.0275 72.1775) (width 0.3) (layer "F.Cu") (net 4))
 (segment (start 135.56 75.09) (end 135.56 76.374) (width 0.3) (layer "F.Cu") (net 4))
 (segment (start 128.78 66.76) (end 127.04 66.76) (width 0.2) (layer "F.Cu") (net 7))
 (segment (start 136.6 66.75) (end 138.25 68.4) (width 0.2) (layer "F.Cu") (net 7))
 (segment (start 135.566 66.75) (end 136.6 66.75) (width 0.2) (layer "F.Cu") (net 7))
 (segment (start 142.33 68.4) (end 142.99 67.74) (width 0.2) (layer "F.Cu") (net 7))
 (segment (start 138.25 68.4) (end 142.33 68.4) (width 0.2) (layer "F.Cu") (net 7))
 (segment (start 142.99 67.74) (end 142.99 64.92) (width 0.2) (layer "F.Cu") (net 7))
 (segment (start 142.99 64.92) (end 141.76 63.69) (width 0.2) (layer "F.Cu") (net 7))
 (segment (start 131.85 63.69) (end 128.78 66.76) (width 0.2) (layer "F.Cu") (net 7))
 (segment (start 141.76 63.69) (end 131.85 63.69) (width 0.2) (layer "F.Cu") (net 7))
 (segment (start 143.27 84.54) (end 144.65 83.16) (width 0.3) (layer "F.Cu") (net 6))
 (segment (start 143.4875 69.6375) (end 140.77 69.6375) (width 0.3) (layer "F.Cu") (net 6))
 (segment (start 124.64 84.54) (end 143.27 84.54) (width 0.3) (layer "F.Cu") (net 6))
 (segment (start 122.65 71.61) (end 122.65 82.55) (width 0.3) (layer "F.Cu") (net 6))
 (segment (start 144.65 83.16) (end 144.65 70.8) (width 0.3) (layer "F.Cu") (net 6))
 (segment (start 123.1 71.16) (end 122.65 71.61) (width 0.3) (layer "F.Cu") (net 6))
 (segment (start 122.65 82.55) (end 124.64 84.54) (width 0.3) (layer "F.Cu") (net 6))
 (segment (start 144.65 70.8) (end 143.4875 69.6375) (width 0.3) (layer "F.Cu") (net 6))
 (segment (start 127.04 71.16) (end 123.1 71.16) (width 0.3) (layer "F.Cu") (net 6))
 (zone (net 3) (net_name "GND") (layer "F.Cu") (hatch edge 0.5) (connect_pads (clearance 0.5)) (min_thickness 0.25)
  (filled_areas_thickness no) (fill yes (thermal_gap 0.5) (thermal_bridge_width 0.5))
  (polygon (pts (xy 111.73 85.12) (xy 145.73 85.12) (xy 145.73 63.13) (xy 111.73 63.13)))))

